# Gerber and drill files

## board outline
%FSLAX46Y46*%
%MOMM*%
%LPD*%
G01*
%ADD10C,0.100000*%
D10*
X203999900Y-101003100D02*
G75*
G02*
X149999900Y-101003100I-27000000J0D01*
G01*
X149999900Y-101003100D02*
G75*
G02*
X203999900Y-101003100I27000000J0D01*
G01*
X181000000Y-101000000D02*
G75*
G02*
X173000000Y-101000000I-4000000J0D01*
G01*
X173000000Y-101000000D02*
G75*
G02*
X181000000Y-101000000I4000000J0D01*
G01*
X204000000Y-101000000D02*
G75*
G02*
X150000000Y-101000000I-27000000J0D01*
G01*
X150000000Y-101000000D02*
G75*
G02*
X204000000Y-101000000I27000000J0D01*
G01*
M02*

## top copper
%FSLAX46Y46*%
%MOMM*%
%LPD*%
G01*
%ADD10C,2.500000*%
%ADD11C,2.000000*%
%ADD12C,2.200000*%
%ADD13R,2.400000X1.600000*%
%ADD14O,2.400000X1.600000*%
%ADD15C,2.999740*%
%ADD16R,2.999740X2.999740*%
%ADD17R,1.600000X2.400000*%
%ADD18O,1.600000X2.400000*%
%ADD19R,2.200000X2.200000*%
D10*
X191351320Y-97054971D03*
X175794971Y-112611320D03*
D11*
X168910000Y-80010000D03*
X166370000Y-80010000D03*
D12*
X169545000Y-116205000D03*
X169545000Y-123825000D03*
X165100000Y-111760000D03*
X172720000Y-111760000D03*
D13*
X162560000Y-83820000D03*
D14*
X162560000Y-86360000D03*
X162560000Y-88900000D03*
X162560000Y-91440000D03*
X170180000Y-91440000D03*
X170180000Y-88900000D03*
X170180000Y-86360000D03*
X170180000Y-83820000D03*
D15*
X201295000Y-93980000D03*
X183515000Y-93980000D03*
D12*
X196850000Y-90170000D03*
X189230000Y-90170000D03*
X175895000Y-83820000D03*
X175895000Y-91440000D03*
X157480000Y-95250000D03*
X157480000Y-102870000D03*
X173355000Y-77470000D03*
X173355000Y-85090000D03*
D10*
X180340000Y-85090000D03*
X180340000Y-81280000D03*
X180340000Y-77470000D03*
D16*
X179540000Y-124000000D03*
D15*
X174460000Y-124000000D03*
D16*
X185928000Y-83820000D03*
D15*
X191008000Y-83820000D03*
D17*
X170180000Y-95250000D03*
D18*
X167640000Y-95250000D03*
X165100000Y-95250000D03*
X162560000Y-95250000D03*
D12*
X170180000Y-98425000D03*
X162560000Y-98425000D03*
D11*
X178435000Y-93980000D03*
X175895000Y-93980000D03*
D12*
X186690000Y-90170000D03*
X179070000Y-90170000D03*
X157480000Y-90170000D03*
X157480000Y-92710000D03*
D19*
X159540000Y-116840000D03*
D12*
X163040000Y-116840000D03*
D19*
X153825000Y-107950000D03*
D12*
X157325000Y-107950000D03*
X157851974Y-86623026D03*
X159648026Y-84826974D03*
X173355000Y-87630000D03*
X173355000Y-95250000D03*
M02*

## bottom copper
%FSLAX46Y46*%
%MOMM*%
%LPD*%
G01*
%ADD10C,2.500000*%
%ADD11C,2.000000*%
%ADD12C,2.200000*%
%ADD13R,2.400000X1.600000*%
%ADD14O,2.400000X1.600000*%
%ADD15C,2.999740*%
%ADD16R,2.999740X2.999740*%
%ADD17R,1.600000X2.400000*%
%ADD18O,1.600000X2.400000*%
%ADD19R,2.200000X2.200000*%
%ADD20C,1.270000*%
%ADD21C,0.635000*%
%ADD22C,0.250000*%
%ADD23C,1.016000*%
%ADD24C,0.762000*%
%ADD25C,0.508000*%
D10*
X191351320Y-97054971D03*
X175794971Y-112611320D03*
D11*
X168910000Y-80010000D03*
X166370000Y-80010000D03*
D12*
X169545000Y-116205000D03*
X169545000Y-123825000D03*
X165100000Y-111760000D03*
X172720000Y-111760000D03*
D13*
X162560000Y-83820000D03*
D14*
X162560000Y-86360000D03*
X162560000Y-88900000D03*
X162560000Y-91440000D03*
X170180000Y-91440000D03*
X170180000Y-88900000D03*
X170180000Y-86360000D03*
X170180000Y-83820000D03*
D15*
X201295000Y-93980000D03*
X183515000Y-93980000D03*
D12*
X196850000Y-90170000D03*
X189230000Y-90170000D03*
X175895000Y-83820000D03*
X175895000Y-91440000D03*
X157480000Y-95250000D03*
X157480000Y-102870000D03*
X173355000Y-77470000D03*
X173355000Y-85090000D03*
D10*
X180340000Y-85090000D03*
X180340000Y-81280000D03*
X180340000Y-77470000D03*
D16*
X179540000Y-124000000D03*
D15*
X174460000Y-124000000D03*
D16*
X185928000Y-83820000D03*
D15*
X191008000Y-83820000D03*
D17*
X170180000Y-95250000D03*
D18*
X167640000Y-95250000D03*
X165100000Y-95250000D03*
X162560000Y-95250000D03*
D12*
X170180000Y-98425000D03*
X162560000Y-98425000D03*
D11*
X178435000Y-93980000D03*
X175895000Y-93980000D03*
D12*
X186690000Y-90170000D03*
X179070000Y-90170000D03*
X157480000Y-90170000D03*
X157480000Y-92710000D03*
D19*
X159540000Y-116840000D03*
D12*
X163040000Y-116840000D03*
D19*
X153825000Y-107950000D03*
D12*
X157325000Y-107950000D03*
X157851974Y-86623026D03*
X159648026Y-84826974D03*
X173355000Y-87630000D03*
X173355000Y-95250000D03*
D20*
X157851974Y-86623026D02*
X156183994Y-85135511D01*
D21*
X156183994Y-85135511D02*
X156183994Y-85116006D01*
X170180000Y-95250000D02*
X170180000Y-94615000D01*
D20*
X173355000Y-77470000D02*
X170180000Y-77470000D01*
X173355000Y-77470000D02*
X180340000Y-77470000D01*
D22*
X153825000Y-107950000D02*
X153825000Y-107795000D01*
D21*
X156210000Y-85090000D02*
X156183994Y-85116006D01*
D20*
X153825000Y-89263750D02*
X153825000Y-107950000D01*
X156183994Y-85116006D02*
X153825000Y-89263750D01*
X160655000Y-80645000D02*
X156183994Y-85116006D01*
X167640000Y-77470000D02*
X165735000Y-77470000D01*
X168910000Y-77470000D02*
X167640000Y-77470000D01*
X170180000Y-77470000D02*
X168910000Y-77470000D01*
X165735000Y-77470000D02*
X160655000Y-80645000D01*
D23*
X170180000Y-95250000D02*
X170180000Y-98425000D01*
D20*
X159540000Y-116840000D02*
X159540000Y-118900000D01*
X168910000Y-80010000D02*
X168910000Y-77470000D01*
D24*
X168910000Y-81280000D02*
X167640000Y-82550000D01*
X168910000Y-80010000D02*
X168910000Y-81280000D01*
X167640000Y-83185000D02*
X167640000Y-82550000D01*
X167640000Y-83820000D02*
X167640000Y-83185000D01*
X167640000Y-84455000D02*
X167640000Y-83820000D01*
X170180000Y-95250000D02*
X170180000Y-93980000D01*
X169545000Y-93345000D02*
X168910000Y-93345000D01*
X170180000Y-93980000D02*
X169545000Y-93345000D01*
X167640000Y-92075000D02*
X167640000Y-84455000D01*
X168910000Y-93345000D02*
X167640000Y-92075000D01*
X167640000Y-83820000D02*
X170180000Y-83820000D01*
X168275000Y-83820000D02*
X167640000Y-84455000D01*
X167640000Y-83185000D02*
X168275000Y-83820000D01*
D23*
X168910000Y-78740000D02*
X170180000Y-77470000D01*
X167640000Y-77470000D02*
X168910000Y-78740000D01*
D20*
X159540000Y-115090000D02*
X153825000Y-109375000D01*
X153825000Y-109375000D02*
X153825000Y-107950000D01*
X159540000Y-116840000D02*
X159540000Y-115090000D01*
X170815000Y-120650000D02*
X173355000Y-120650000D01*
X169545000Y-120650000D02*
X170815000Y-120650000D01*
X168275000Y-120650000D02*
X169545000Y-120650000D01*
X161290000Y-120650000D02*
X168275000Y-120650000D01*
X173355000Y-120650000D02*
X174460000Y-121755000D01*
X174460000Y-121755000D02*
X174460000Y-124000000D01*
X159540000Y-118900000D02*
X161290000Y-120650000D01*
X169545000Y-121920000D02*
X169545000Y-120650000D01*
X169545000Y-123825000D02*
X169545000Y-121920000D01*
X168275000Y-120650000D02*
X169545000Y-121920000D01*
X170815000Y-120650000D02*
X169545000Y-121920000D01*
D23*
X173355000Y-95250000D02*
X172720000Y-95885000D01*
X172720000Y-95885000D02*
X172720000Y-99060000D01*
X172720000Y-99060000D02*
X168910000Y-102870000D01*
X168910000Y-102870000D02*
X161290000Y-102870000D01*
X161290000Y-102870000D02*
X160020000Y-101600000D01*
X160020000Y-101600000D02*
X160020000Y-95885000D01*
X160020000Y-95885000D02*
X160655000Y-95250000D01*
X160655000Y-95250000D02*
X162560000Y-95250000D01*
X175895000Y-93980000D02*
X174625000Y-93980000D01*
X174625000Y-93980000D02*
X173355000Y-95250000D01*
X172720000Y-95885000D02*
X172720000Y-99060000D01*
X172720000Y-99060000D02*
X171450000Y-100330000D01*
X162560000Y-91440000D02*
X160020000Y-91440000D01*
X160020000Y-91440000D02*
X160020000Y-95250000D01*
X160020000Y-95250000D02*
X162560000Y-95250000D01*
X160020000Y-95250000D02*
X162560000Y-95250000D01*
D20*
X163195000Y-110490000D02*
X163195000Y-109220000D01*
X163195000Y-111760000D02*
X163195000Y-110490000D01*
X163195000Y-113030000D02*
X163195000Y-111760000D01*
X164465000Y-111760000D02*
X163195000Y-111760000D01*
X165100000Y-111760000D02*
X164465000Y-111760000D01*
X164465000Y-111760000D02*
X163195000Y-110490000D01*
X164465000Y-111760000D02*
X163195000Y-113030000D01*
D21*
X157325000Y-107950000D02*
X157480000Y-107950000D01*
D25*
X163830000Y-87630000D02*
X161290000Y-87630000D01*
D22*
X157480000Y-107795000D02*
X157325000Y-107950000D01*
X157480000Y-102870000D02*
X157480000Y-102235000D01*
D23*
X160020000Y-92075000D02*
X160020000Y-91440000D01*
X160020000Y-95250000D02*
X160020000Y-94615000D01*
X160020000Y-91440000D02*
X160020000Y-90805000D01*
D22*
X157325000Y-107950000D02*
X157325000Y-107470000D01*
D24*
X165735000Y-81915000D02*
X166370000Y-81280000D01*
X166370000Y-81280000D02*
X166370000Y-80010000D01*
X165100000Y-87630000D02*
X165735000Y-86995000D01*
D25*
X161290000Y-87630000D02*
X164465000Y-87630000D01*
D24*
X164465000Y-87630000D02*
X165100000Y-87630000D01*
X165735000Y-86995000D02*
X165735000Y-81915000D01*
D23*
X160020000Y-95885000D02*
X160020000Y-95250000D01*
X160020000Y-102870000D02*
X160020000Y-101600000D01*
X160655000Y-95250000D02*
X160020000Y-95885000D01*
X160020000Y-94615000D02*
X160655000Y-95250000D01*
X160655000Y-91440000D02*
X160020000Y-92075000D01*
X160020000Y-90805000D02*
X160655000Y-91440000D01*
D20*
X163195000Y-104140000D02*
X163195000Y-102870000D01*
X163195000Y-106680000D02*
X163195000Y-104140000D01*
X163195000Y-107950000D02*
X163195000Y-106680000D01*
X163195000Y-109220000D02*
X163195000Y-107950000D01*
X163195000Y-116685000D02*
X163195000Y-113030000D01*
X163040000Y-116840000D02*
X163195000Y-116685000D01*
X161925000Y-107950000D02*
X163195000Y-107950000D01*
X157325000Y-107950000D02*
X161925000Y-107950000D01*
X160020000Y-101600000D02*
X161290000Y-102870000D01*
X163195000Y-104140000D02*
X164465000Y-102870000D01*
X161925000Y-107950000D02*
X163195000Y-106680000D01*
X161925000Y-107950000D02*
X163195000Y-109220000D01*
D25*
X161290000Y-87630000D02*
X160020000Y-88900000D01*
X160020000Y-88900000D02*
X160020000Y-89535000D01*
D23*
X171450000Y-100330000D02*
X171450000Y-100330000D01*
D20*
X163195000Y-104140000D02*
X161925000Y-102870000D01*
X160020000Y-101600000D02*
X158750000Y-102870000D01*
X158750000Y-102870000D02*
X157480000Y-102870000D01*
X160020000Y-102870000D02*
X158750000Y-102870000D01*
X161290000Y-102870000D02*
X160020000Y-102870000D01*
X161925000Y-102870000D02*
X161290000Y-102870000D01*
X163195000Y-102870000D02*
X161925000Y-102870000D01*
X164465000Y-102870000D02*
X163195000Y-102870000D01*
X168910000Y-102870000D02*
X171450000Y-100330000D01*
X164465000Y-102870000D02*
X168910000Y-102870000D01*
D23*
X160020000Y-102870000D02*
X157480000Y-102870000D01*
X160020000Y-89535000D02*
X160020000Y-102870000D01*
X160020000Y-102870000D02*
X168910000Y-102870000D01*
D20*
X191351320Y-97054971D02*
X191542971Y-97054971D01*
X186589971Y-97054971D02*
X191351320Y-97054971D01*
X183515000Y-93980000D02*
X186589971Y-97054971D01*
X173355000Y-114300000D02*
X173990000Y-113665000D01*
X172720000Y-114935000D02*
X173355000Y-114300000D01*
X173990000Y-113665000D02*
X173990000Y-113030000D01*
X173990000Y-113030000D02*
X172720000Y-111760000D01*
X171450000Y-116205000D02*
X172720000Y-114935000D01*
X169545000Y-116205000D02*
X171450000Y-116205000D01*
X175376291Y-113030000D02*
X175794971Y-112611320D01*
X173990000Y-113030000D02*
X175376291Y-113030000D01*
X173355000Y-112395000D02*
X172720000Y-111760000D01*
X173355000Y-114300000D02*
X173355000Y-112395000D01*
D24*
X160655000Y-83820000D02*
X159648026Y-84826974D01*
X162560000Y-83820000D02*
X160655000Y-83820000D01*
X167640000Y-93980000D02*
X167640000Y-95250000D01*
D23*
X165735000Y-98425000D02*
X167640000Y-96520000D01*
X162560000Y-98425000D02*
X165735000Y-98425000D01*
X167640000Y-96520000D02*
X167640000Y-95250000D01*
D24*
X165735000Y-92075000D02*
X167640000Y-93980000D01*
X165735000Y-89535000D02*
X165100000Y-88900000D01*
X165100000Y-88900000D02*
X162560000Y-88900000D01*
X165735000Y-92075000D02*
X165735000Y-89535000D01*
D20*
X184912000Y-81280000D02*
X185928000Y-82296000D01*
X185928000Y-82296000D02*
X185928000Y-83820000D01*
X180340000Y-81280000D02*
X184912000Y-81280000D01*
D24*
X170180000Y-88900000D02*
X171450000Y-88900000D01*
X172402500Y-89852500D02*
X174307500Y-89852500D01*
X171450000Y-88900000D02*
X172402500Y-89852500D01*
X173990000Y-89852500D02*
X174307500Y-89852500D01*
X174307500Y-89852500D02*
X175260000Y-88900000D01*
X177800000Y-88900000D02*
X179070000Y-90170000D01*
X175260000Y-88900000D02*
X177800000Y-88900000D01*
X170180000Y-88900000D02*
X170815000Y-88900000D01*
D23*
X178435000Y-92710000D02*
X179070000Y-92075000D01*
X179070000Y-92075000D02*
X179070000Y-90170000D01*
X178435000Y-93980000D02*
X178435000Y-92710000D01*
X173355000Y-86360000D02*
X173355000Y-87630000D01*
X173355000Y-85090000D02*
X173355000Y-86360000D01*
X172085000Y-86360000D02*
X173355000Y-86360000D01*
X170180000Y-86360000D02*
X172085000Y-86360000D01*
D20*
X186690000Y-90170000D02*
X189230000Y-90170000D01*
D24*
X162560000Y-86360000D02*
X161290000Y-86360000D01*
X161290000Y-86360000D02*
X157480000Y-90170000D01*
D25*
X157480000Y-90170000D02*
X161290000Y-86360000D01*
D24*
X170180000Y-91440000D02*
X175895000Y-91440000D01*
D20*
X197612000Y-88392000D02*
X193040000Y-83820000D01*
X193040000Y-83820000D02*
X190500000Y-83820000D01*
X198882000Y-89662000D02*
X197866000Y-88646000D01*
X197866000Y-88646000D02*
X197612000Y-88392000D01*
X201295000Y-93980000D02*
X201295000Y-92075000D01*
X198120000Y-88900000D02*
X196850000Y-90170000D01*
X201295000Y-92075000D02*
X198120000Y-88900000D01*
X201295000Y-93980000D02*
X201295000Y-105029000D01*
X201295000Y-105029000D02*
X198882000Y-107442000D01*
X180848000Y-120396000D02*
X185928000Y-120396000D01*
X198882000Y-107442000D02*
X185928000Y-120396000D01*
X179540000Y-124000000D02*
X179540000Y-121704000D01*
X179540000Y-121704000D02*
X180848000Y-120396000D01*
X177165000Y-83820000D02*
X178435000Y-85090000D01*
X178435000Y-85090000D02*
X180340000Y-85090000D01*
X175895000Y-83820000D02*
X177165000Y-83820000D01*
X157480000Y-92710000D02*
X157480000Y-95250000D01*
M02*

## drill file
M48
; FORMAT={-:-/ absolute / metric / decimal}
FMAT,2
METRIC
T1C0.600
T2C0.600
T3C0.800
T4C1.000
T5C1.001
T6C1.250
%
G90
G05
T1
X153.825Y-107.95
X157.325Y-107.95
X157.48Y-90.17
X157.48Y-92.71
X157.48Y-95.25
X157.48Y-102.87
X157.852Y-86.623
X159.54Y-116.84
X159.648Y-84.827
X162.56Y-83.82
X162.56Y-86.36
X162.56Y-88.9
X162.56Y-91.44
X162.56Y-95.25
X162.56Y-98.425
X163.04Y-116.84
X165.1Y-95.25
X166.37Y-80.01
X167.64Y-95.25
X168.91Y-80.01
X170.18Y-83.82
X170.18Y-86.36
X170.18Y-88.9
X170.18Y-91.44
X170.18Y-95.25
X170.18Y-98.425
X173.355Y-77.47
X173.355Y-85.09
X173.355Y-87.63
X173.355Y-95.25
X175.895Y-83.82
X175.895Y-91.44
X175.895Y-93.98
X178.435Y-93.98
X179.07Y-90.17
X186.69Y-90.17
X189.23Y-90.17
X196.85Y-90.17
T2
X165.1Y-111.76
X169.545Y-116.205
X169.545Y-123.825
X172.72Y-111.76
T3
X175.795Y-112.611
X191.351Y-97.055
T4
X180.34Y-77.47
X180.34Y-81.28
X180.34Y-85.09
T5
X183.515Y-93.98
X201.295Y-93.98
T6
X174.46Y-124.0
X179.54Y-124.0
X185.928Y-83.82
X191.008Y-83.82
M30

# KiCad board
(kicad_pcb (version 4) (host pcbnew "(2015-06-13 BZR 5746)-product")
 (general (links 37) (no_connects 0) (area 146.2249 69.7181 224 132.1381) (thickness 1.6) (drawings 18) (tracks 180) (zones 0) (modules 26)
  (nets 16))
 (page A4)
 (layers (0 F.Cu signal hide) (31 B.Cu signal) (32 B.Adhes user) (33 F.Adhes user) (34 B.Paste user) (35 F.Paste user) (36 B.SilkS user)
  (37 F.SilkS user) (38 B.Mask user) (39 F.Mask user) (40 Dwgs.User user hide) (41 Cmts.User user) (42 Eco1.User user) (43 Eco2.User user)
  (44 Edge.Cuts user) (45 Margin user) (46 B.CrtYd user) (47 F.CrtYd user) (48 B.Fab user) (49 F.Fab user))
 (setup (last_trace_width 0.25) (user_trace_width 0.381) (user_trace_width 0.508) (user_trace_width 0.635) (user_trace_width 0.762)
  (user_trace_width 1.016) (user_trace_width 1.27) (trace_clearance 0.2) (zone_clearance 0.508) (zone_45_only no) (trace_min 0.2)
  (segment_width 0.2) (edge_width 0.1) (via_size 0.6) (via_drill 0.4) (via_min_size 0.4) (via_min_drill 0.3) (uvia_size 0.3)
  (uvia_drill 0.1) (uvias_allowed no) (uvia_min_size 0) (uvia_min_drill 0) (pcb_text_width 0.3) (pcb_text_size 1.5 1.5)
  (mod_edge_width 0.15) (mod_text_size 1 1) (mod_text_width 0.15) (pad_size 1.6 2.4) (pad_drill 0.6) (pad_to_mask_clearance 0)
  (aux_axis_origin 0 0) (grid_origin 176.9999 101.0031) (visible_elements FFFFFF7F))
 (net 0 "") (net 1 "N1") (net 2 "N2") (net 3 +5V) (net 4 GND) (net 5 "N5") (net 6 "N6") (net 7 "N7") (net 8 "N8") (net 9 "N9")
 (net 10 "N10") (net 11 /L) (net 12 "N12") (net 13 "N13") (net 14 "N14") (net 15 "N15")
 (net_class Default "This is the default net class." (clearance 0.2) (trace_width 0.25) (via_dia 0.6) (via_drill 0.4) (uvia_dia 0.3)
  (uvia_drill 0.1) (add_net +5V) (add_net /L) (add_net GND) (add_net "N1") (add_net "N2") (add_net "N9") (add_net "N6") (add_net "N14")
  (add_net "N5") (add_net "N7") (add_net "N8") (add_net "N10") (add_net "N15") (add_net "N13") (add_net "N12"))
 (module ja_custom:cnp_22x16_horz (layer F.Cu) (at 189.23 110.49 225)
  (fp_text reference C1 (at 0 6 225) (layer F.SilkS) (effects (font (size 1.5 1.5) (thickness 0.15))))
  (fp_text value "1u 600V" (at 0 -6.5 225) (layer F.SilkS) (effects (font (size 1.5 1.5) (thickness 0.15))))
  (pad 1 thru_hole circle (at -11 8 225) (size 2.5 2.5) (drill 0.8) (layers *.Cu *.Mask F.SilkS) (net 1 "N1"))
  (pad 2 thru_hole circle (at 11 8 225) (size 2.5 2.5) (drill 0.8) (layers *.Cu *.Mask F.SilkS) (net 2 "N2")))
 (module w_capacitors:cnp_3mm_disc (layer F.Cu) (at 167.64 80.01 180)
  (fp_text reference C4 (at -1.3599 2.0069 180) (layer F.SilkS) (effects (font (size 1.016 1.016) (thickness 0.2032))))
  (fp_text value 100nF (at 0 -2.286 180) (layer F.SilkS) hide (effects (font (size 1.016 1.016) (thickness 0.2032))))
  (pad 1 thru_hole circle (at -1.27 0 180) (size 2 2) (drill 0.6) (layers *.Cu *.Mask F.SilkS) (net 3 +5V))
  (pad 2 thru_hole circle (at 1.27 0 180) (size 2 2) (drill 0.6) (layers *.Cu *.Mask F.SilkS) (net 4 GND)))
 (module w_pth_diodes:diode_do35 (layer F.Cu) (at 169.545 120.015 270)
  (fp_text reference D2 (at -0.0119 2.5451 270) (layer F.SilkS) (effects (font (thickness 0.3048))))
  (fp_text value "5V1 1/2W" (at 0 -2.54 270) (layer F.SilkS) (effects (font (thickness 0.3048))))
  (pad 1 thru_hole circle (at -3.81 0 270) (size 2.2 2.2) (drill 0.6001) (layers *.Cu *.Mask F.SilkS) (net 2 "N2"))
  (pad 2 thru_hole circle (at 3.81 0 270) (size 2.2 2.2) (drill 0.6001) (layers *.Cu *.Mask F.SilkS) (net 3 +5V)))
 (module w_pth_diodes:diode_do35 (layer F.Cu) (at 168.91 111.76)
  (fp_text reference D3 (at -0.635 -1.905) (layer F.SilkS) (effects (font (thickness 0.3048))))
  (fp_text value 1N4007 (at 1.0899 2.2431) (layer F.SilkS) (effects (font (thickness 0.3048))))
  (pad 1 thru_hole circle (at -3.81 0) (size 2.2 2.2) (drill 0.6001) (layers *.Cu *.Mask F.SilkS) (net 4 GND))
  (pad 2 thru_hole circle (at 3.81 0) (size 2.2 2.2) (drill 0.6001) (layers *.Cu *.Mask F.SilkS) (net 2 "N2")))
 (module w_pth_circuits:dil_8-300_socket (layer F.Cu) (at 166.37 87.63 270)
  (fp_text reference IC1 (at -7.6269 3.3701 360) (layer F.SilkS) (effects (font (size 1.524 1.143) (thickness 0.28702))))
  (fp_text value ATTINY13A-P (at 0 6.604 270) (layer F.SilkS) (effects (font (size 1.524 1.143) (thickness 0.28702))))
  (pad 1 thru_hole rect (at -3.81 3.81 270) (size 1.6 2.4) (drill 0.6) (layers *.Cu *.Mask F.SilkS) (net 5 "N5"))
  (pad 2 thru_hole oval (at -1.27 3.81 270) (size 1.6 2.4) (drill 0.6) (layers *.Cu *.Mask F.SilkS) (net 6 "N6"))
  (pad 3 thru_hole oval (at 1.27 3.81 270) (size 1.6 2.4) (drill 0.6) (layers *.Cu *.Mask F.SilkS) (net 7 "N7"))
  (pad 4 thru_hole oval (at 3.81 3.81 270) (size 1.6 2.4) (drill 0.6) (layers *.Cu *.Mask F.SilkS) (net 4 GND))
  (pad 5 thru_hole oval (at 3.81 -3.81 270) (size 1.6 2.4) (drill 0.6) (layers *.Cu *.Mask F.SilkS) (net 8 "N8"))
  (pad 6 thru_hole oval (at 1.27 -3.81 270) (size 1.6 2.4) (drill 0.6) (layers *.Cu *.Mask F.SilkS) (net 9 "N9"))
  (pad 7 thru_hole oval (at -1.27 -3.81 270) (size 1.6 2.4) (drill 0.6) (layers *.Cu *.Mask F.SilkS) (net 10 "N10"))
  (pad 8 thru_hole oval (at -3.81 -3.81 270) (size 1.6 2.4) (drill 0.6) (layers *.Cu *.Mask F.SilkS) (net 3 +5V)))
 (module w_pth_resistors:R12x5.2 (layer F.Cu) (at 192.405 93.98 180) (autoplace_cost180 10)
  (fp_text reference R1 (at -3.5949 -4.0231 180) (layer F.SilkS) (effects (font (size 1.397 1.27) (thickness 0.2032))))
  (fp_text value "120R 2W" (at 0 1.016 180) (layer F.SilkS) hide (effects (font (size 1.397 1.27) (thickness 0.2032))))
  (pad 1 thru_hole circle (at -8.89 0 180) (size 2.99974 2.99974) (drill 1.00076) (layers *.Cu *.Mask F.SilkS) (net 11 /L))
  (pad 2 thru_hole circle (at 8.89 0 180) (size 2.99974 2.99974) (drill 1.00076) (layers *.Cu *.Mask F.SilkS) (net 1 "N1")))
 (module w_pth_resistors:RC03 (layer F.Cu) (at 193.04 90.17 180) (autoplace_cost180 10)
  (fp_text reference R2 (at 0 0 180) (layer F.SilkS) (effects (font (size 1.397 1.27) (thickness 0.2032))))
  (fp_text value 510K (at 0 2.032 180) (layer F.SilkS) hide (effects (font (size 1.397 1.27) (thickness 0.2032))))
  (pad 1 thru_hole circle (at -3.81 0 180) (size 2.2 2.2) (drill 0.6) (layers *.Cu *.Mask F.SilkS) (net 11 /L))
  (pad 2 thru_hole circle (at 3.81 0 180) (size 2.2 2.2) (drill 0.6) (layers *.Cu *.Mask F.SilkS) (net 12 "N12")))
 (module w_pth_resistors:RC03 (layer F.Cu) (at 175.895 87.63 270) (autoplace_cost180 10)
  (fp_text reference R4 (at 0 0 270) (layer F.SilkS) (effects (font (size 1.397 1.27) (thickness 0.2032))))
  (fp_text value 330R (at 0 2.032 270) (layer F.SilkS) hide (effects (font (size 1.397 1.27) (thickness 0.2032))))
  (pad 1 thru_hole circle (at -3.81 0 270) (size 2.2 2.2) (drill 0.6) (layers *.Cu *.Mask F.SilkS) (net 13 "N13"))
  (pad 2 thru_hole circle (at 3.81 0 270) (size 2.2 2.2) (drill 0.6) (layers *.Cu *.Mask F.SilkS) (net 8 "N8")))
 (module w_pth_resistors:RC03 (layer F.Cu) (at 157.48 99.06 270) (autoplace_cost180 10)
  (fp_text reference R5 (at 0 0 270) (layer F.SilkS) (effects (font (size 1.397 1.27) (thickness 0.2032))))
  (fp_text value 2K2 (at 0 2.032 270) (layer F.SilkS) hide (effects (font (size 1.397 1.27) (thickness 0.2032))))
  (pad 1 thru_hole circle (at -3.81 0 270) (size 2.2 2.2) (drill 0.6) (layers *.Cu *.Mask F.SilkS) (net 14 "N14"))
  (pad 2 thru_hole circle (at 3.81 0 270) (size 2.2 2.2) (drill 0.6) (layers *.Cu *.Mask F.SilkS) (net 4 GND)))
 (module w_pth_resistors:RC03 (layer F.Cu) (at 173.355 81.28 270) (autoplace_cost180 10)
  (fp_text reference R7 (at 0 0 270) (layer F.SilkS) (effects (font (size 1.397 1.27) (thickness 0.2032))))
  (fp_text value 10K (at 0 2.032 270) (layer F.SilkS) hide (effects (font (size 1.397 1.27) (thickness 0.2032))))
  (pad 1 thru_hole circle (at -3.81 0 270) (size 2.2 2.2) (drill 0.6) (layers *.Cu *.Mask F.SilkS) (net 3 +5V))
  (pad 2 thru_hole circle (at 3.81 0 270) (size 2.2 2.2) (drill 0.6) (layers *.Cu *.Mask F.SilkS) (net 10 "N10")))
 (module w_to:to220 (layer F.Cu) (at 180.34 81.28 270)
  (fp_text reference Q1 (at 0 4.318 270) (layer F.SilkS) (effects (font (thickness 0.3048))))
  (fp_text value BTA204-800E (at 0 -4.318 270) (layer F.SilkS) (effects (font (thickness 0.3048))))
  (pad 1 thru_hole circle (at 3.81 0 270) (size 2.5 2.5) (drill 1) (layers *.Cu *.Mask F.SilkS) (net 13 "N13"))
  (pad 2 thru_hole circle (at 0 0 270) (size 2.5 2.5) (drill 1) (layers *.Cu *.Mask F.SilkS) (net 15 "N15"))
  (pad 3 thru_hole circle (at -3.81 0 270) (size 2.5 2.5) (drill 1) (layers *.Cu *.Mask F.SilkS) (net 3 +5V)))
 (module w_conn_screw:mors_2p (layer F.Cu) (at 177 124 180)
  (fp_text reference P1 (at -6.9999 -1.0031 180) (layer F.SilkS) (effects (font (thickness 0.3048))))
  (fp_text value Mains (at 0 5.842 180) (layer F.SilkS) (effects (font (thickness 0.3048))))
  (pad 1 thru_hole rect (at -2.54 0 180) (size 2.99974 2.99974) (drill 1.24968) (layers *.Cu *.Mask F.SilkS) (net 11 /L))
  (pad 2 thru_hole circle (at 2.54 0 180) (size 2.99974 2.99974) (drill 1.24968) (layers *.Cu *.Mask F.SilkS) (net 3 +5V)))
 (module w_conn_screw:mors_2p (layer F.Cu) (at 188.468 83.82)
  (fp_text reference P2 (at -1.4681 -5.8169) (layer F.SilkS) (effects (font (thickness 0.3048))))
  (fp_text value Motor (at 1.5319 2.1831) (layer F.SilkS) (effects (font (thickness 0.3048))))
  (pad 1 thru_hole rect (at -2.54 0) (size 2.99974 2.99974) (drill 1.24968) (layers *.Cu *.Mask F.SilkS) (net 15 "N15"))
  (pad 2 thru_hole circle (at 2.54 0) (size 2.99974 2.99974) (drill 1.24968) (layers *.Cu *.Mask F.SilkS) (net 11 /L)))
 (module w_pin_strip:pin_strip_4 (layer F.Cu) (at 166.37 95.25 180)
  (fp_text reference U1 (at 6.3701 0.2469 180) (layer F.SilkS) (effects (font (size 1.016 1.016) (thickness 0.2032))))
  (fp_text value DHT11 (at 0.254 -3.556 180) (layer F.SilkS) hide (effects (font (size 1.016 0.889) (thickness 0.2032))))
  (pad 1 thru_hole rect (at -3.81 0 180) (size 1.6 2.4) (drill 0.6) (layers *.Cu *.Mask F.SilkS) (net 3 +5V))
  (pad 2 thru_hole oval (at -1.27 0 180) (size 1.6 2.4) (drill 0.6) (layers *.Cu *.Mask F.SilkS) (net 7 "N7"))
  (pad 3 thru_hole oval (at 1.27 0 180) (size 1.6 2.4) (drill 0.6) (layers *.Cu *.Mask F.SilkS))
  (pad 4 thru_hole oval (at 3.81 0 180) (size 1.6 2.4) (drill 0.6) (layers *.Cu *.Mask F.SilkS) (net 4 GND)))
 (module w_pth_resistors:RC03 (layer F.Cu) (at 166.37 98.425 180) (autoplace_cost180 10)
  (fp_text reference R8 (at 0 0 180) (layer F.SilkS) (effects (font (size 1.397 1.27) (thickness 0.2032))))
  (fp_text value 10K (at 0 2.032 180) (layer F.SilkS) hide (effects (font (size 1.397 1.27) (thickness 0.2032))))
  (pad 1 thru_hole circle (at -3.81 0 180) (size 2.2 2.2) (drill 0.6) (layers *.Cu *.Mask F.SilkS) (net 3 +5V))
  (pad 2 thru_hole circle (at 3.81 0 180) (size 2.2 2.2) (drill 0.6) (layers *.Cu *.Mask F.SilkS) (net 7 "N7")))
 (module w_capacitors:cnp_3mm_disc (layer F.Cu) (at 177.165 93.98 180)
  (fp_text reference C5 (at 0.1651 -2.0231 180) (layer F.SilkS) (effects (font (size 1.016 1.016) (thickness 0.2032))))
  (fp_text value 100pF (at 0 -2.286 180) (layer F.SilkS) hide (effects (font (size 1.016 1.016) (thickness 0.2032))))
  (pad 1 thru_hole circle (at -1.27 0 180) (size 2 2) (drill 0.6) (layers *.Cu *.Mask F.SilkS) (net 9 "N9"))
  (pad 2 thru_hole circle (at 1.27 0 180) (size 2 2) (drill 0.6) (layers *.Cu *.Mask F.SilkS) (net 4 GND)))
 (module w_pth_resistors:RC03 (layer F.Cu) (at 182.88 90.17 180) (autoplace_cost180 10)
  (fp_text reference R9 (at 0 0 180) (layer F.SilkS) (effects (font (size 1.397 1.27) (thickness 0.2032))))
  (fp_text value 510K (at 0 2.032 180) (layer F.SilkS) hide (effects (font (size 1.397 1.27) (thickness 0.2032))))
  (pad 1 thru_hole circle (at -3.81 0 180) (size 2.2 2.2) (drill 0.6) (layers *.Cu *.Mask F.SilkS) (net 12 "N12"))
  (pad 2 thru_hole circle (at 3.81 0 180) (size 2.2 2.2) (drill 0.6) (layers *.Cu *.Mask F.SilkS) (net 9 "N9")))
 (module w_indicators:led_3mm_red (layer F.Cu) (at 157.48 91.44)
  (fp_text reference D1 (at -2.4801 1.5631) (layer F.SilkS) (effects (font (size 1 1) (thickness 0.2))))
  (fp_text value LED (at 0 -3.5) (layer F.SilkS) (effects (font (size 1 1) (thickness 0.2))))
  (pad 1 thru_hole circle (at 0 -1.27) (size 2.2 2.2) (drill 0.6) (layers *.Cu *.Mask F.SilkS) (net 6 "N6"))
  (pad 2 thru_hole circle (at 0 1.27) (size 2.2 2.2) (drill 0.6) (layers *.Cu *.Mask F.SilkS) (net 14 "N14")))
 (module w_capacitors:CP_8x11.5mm (layer F.Cu) (at 161.29 116.84 270)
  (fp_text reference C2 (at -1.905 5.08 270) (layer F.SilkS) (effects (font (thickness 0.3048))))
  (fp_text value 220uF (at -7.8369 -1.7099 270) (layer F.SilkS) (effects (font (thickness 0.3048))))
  (pad 1 thru_hole rect (at 0 1.75 270) (size 2.2 2.2) (drill 0.6) (layers *.Cu *.Mask F.SilkS) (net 3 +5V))
  (pad 2 thru_hole circle (at 0 -1.75 270) (size 2.2 2.2) (drill 0.6) (layers *.Cu *.Mask F.SilkS) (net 4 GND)))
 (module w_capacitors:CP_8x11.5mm (layer F.Cu) (at 155.575 107.95 270)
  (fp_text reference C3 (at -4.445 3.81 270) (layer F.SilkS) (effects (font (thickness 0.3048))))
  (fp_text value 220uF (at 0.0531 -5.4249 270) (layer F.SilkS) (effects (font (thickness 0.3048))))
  (pad 1 thru_hole rect (at 0 1.75 270) (size 2.2 2.2) (drill 0.6) (layers *.Cu *.Mask F.SilkS) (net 3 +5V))
  (pad 2 thru_hole circle (at 0 -1.75 270) (size 2.2 2.2) (drill 0.6) (layers *.Cu *.Mask F.SilkS) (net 4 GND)))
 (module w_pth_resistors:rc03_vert (layer F.Cu) (at 158.75 85.725 45)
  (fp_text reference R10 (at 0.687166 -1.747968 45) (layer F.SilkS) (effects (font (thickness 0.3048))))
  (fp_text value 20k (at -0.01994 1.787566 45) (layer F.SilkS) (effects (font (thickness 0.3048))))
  (pad 1 thru_hole circle (at -1.270001 0 45) (size 2.2 2.2) (drill 0.6) (layers *.Cu *.Mask F.SilkS) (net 3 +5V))
  (pad 2 thru_hole circle (at 1.27 0 45) (size 2.2 2.2) (drill 0.6) (layers *.Cu *.Mask F.SilkS) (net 5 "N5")))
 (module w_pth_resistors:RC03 (layer F.Cu) (at 173.355 91.44 270) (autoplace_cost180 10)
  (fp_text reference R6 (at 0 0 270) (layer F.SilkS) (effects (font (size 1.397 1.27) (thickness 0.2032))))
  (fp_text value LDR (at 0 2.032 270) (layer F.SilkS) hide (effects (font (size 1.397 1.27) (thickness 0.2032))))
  (pad 1 thru_hole circle (at -3.81 0 270) (size 2.2 2.2) (drill 0.6) (layers *.Cu *.Mask F.SilkS) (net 10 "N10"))
  (pad 2 thru_hole circle (at 3.81 0 270) (size 2.2 2.2) (drill 0.6) (layers *.Cu *.Mask F.SilkS) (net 4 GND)))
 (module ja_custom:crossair (layer F.Cu) (at 202.9999 75.0031)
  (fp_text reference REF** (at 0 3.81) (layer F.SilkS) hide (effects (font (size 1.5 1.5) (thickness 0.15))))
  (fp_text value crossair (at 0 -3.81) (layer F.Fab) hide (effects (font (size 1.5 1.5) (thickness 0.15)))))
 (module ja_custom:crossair (layer F.Cu) (at 150.9999 75.0031)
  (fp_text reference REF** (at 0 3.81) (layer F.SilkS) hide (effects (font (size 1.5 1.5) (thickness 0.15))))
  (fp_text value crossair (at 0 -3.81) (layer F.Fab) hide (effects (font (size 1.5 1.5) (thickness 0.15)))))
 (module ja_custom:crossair (layer F.Cu) (at 150.9999 127.0031)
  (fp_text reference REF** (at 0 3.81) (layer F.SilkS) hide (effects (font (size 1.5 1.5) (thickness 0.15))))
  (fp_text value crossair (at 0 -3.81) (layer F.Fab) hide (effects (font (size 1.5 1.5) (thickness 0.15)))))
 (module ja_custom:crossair (layer F.Cu) (at 202.9999 127.0031)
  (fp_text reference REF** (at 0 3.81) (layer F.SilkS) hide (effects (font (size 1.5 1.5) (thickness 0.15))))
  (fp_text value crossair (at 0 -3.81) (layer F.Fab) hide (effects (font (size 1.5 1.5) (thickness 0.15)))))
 (gr_circle (center 176.9999 101.0031) (end 203.9999 101.0031) (layer Edge.Cuts) (width 0.1))
 (gr_circle (center 177 101) (end 181 101) (layer Edge.Cuts) (width 0.1))
 (gr_circle (center 177 101) (end 204 101) (layer Edge.Cuts) (width 0.1))
 (segment (start 157.851974 86.623026) (end 156.183994 85.135511) (width 1.27) (layer B.Cu) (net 3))
 (segment (start 156.183994 85.135511) (end 156.183994 85.116006) (width 0.635) (layer B.Cu) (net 3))
 (segment (start 170.18 95.25) (end 170.18 94.615) (width 0.635) (layer B.Cu) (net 3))
 (segment (start 173.355 77.47) (end 170.18 77.47) (width 1.27) (layer B.Cu) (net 3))
 (segment (start 173.355 77.47) (end 180.34 77.47) (width 1.27) (layer B.Cu) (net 3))
 (segment (start 153.825 107.95) (end 153.825 107.795) (width 0.25) (layer B.Cu) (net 3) (status 30))
 (segment (start 156.21 85.09) (end 156.183994 85.116006) (width 0.635) (layer B.Cu) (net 3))
 (segment (start 153.825 89.26375) (end 153.825 107.95) (width 1.27) (layer B.Cu) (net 3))
 (segment (start 156.183994 85.116006) (end 153.825 89.26375) (width 1.27) (layer B.Cu) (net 3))
 (segment (start 160.655 80.645) (end 156.183994 85.116006) (width 1.27) (layer B.Cu) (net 3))
 (segment (start 167.64 77.47) (end 165.735 77.47) (width 1.27) (layer B.Cu) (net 3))
 (segment (start 168.91 77.47) (end 167.64 77.47) (width 1.27) (layer B.Cu) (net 3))
 (segment (start 170.18 77.47) (end 168.91 77.47) (width 1.27) (layer B.Cu) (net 3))
 (segment (start 165.735 77.47) (end 160.655 80.645) (width 1.27) (layer B.Cu) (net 3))
 (segment (start 170.18 95.25) (end 170.18 98.425) (width 1.016) (layer B.Cu) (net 3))
 (segment (start 159.54 116.84) (end 159.54 118.9) (width 1.27) (layer B.Cu) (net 3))
 (segment (start 168.91 80.01) (end 168.91 77.47) (width 1.27) (layer B.Cu) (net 3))
 (segment (start 168.91 81.28) (end 167.64 82.55) (width 0.762) (layer B.Cu) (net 3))
 (segment (start 168.91 80.01) (end 168.91 81.28) (width 0.762) (layer B.Cu) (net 3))
 (segment (start 167.64 83.185) (end 167.64 82.55) (width 0.762) (layer B.Cu) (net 3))
 (segment (start 167.64 83.82) (end 167.64 83.185) (width 0.762) (layer B.Cu) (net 3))
 (segment (start 167.64 84.455) (end 167.64 83.82) (width 0.762) (layer B.Cu) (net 3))
 (segment (start 170.18 95.25) (end 170.18 93.98) (width 0.762) (layer B.Cu) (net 3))
 (segment (start 169.545 93.345) (end 168.91 93.345) (width 0.762) (layer B.Cu) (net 3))
 (segment (start 170.18 93.98) (end 169.545 93.345) (width 0.762) (layer B.Cu) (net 3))
 (segment (start 167.64 92.075) (end 167.64 84.455) (width 0.762) (layer B.Cu) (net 3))
 (segment (start 168.91 93.345) (end 167.64 92.075) (width 0.762) (layer B.Cu) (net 3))
 (segment (start 167.64 83.82) (end 170.18 83.82) (width 0.762) (layer B.Cu) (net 3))
 (segment (start 168.275 83.82) (end 167.64 84.455) (width 0.762) (layer B.Cu) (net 3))
 (segment (start 167.64 83.185) (end 168.275 83.82) (width 0.762) (layer B.Cu) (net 3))
 (segment (start 168.91 78.74) (end 170.18 77.47) (width 1.016) (layer B.Cu) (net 3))
 (segment (start 167.64 77.47) (end 168.91 78.74) (width 1.016) (layer B.Cu) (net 3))
 (segment (start 159.54 115.09) (end 153.825 109.375) (width 1.27) (layer B.Cu) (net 3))
 (segment (start 153.825 109.375) (end 153.825 107.95) (width 1.27) (layer B.Cu) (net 3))
 (segment (start 159.54 116.84) (end 159.54 115.09) (width 1.27) (layer B.Cu) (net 3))
 (segment (start 170.815 120.65) (end 173.355 120.65) (width 1.27) (layer B.Cu) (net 3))
 (segment (start 169.545 120.65) (end 170.815 120.65) (width 1.27) (layer B.Cu) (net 3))
 (segment (start 168.275 120.65) (end 169.545 120.65) (width 1.27) (layer B.Cu) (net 3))
 (segment (start 161.29 120.65) (end 168.275 120.65) (width 1.27) (layer B.Cu) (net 3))
 (segment (start 173.355 120.65) (end 174.46 121.755) (width 1.27) (layer B.Cu) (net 3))
 (segment (start 174.46 121.755) (end 174.46 124) (width 1.27) (layer B.Cu) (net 3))
 (segment (start 159.54 118.9) (end 161.29 120.65) (width 1.27) (layer B.Cu) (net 3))
 (segment (start 169.545 121.92) (end 169.545 120.65) (width 1.27) (layer B.Cu) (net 3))
 (segment (start 169.545 123.825) (end 169.545 121.92) (width 1.27) (layer B.Cu) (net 3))
 (segment (start 168.275 120.65) (end 169.545 121.92) (width 1.27) (layer B.Cu) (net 3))
 (segment (start 170.815 120.65) (end 169.545 121.92) (width 1.27) (layer B.Cu) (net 3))
 (segment (start 173.355 95.25) (end 172.72 95.885) (width 1.016) (layer B.Cu) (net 4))
 (segment (start 172.72 95.885) (end 172.72 99.06) (width 1.016) (layer B.Cu) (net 4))
 (segment (start 172.72 99.06) (end 168.91 102.87) (width 1.016) (layer B.Cu) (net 4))
 (segment (start 168.91 102.87) (end 161.29 102.87) (width 1.016) (layer B.Cu) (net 4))
 (segment (start 161.29 102.87) (end 160.02 101.6) (width 1.016) (layer B.Cu) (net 4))
 (segment (start 160.02 101.6) (end 160.02 95.885) (width 1.016) (layer B.Cu) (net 4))
 (segment (start 160.02 95.885) (end 160.655 95.25) (width 1.016) (layer B.Cu) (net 4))
 (segment (start 160.655 95.25) (end 162.56 95.25) (width 1.016) (layer B.Cu) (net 4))
 (segment (start 175.895 93.98) (end 174.625 93.98) (width 1.016) (layer B.Cu) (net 4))
 (segment (start 174.625 93.98) (end 173.355 95.25) (width 1.016) (layer B.Cu) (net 4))
 (segment (start 172.72 95.885) (end 172.72 99.06) (width 1.016) (layer B.Cu) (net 4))
 (segment (start 172.72 99.06) (end 171.45 100.33) (width 1.016) (layer B.Cu) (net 4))
 (segment (start 162.56 91.44) (end 160.02 91.44) (width 1.016) (layer B.Cu) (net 4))
 (segment (start 160.02 91.44) (end 160.02 95.25) (width 1.016) (layer B.Cu) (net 4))
 (segment (start 160.02 95.25) (end 162.56 95.25) (width 1.016) (layer B.Cu) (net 4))
 (segment (start 160.02 95.25) (end 162.56 95.25) (width 1.016) (layer B.Cu) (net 4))
 (segment (start 163.195 110.49) (end 163.195 109.22) (width 1.27) (layer B.Cu) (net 4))
 (segment (start 163.195 111.76) (end 163.195 110.49) (width 1.27) (layer B.Cu) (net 4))
 (segment (start 163.195 113.03) (end 163.195 111.76) (width 1.27) (layer B.Cu) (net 4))
 (segment (start 164.465 111.76) (end 163.195 111.76) (width 1.27) (layer B.Cu) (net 4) (status 10))
 (segment (start 165.1 111.76) (end 164.465 111.76) (width 1.27) (layer B.Cu) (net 4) (status 10))
 (segment (start 164.465 111.76) (end 163.195 110.49) (width 1.27) (layer B.Cu) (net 4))
 (segment (start 164.465 111.76) (end 163.195 113.03) (width 1.27) (layer B.Cu) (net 4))
 (segment (start 157.325 107.95) (end 157.48 107.95) (width 0.635) (layer B.Cu) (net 4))
 (segment (start 163.83 87.63) (end 161.29 87.63) (width 0.508) (layer B.Cu) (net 4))
 (segment (start 157.48 107.795) (end 157.325 107.95) (width 0.25) (layer B.Cu) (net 4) (status 30))
 (segment (start 157.48 102.87) (end 157.48 102.235) (width 0.25) (layer B.Cu) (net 4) (status 30))
 (segment (start 160.02 92.075) (end 160.02 91.44) (width 1.016) (layer B.Cu) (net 4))
 (segment (start 160.02 95.25) (end 160.02 94.615) (width 1.016) (layer B.Cu) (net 4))
 (segment (start 160.02 91.44) (end 160.02 90.805) (width 1.016) (layer B.Cu) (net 4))
 (segment (start 157.325 107.95) (end 157.325 107.47) (width 0.25) (layer B.Cu) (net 4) (status 30))
 (segment (start 165.735 81.915) (end 166.37 81.28) (width 0.762) (layer B.Cu) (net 4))
 (segment (start 166.37 81.28) (end 166.37 80.01) (width 0.762) (layer B.Cu) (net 4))
 (segment (start 165.1 87.63) (end 165.735 86.995) (width 0.762) (layer B.Cu) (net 4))
 (segment (start 161.29 87.63) (end 164.465 87.63) (width 0.508) (layer B.Cu) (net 4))
 (segment (start 164.465 87.63) (end 165.1 87.63) (width 0.762) (layer B.Cu) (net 4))
 (segment (start 165.735 86.995) (end 165.735 81.915) (width 0.762) (layer B.Cu) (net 4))
 (segment (start 160.02 95.885) (end 160.02 95.25) (width 1.016) (layer B.Cu) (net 4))
 (segment (start 160.02 102.87) (end 160.02 101.6) (width 1.016) (layer B.Cu) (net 4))
 (segment (start 160.655 95.25) (end 160.02 95.885) (width 1.016) (layer B.Cu) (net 4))
 (segment (start 160.02 94.615) (end 160.655 95.25) (width 1.016) (layer B.Cu) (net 4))
 (segment (start 160.655 91.44) (end 160.02 92.075) (width 1.016) (layer B.Cu) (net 4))
 (segment (start 160.02 90.805) (end 160.655 91.44) (width 1.016) (layer B.Cu) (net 4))
 (segment (start 163.195 104.14) (end 163.195 102.87) (width 1.27) (layer B.Cu) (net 4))
 (segment (start 163.195 106.68) (end 163.195 104.14) (width 1.27) (layer B.Cu) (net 4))
 (segment (start 163.195 107.95) (end 163.195 106.68) (width 1.27) (layer B.Cu) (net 4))
 (segment (start 163.195 109.22) (end 163.195 107.95) (width 1.27) (layer B.Cu) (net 4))
 (segment (start 163.195 116.685) (end 163.195 113.03) (width 1.27) (layer B.Cu) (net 4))
 (segment (start 163.04 116.84) (end 163.195 116.685) (width 1.27) (layer B.Cu) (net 4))
 (segment (start 161.925 107.95) (end 163.195 107.95) (width 1.27) (layer B.Cu) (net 4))
 (segment (start 157.325 107.95) (end 161.925 107.95) (width 1.27) (layer B.Cu) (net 4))
 (segment (start 160.02 101.6) (end 161.29 102.87) (width 1.27) (layer B.Cu) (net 4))
 (segment (start 163.195 104.14) (end 164.465 102.87) (width 1.27) (layer B.Cu) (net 4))
 (segment (start 161.925 107.95) (end 163.195 106.68) (width 1.27) (layer B.Cu) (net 4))
 (segment (start 161.925 107.95) (end 163.195 109.22) (width 1.27) (layer B.Cu) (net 4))
 (segment (start 161.29 87.63) (end 160.02 88.9) (width 0.508) (layer B.Cu) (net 4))
 (segment (start 160.02 88.9) (end 160.02 89.535) (width 0.508) (layer B.Cu) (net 4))
 (segment (start 171.45 100.33) (end 171.45 100.33) (width 1.016) (layer B.Cu) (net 4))
 (segment (start 163.195 104.14) (end 161.925 102.87) (width 1.27) (layer B.Cu) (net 4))
 (segment (start 160.02 101.6) (end 158.75 102.87) (width 1.27) (layer B.Cu) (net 4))
 (segment (start 158.75 102.87) (end 157.48 102.87) (width 1.27) (layer B.Cu) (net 4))
 (segment (start 160.02 102.87) (end 158.75 102.87) (width 1.27) (layer B.Cu) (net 4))
 (segment (start 161.29 102.87) (end 160.02 102.87) (width 1.27) (layer B.Cu) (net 4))
 (segment (start 161.925 102.87) (end 161.29 102.87) (width 1.27) (layer B.Cu) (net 4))
 (segment (start 163.195 102.87) (end 161.925 102.87) (width 1.27) (layer B.Cu) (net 4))
 (segment (start 164.465 102.87) (end 163.195 102.87) (width 1.27) (layer B.Cu) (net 4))
 (segment (start 168.91 102.87) (end 171.45 100.33) (width 1.27) (layer B.Cu) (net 4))
 (segment (start 164.465 102.87) (end 168.91 102.87) (width 1.27) (layer B.Cu) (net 4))
 (segment (start 160.02 102.87) (end 157.48 102.87) (width 1.016) (layer B.Cu) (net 4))
 (segment (start 160.02 89.535) (end 160.02 102.87) (width 1.016) (layer B.Cu) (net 4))
 (segment (start 160.02 102.87) (end 168.91 102.87) (width 1.016) (layer B.Cu) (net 4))
 (segment (start 191.35132 97.054971) (end 191.542971 97.054971) (width 1.27) (layer B.Cu) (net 1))
 (segment (start 186.589971 97.054971) (end 191.35132 97.054971) (width 1.27) (layer B.Cu) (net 1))
 (segment (start 183.515 93.98) (end 186.589971 97.054971) (width 1.27) (layer B.Cu) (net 1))
 (segment (start 173.355 114.3) (end 173.99 113.665) (width 1.27) (layer B.Cu) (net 2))
 (segment (start 172.72 114.935) (end 173.355 114.3) (width 1.27) (layer B.Cu) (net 2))
 (segment (start 173.99 113.665) (end 173.99 113.03) (width 1.27) (layer B.Cu) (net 2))
 (segment (start 173.99 113.03) (end 172.72 111.76) (width 1.27) (layer B.Cu) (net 2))
 (segment (start 171.45 116.205) (end 172.72 114.935) (width 1.27) (layer B.Cu) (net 2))
 (segment (start 169.545 116.205) (end 171.45 116.205) (width 1.27) (layer B.Cu) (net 2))
 (segment (start 175.376291 113.03) (end 175.794971 112.61132) (width 1.27) (layer B.Cu) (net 2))
 (segment (start 173.99 113.03) (end 175.376291 113.03) (width 1.27) (layer B.Cu) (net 2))
 (segment (start 173.355 112.395) (end 172.72 111.76) (width 1.27) (layer B.Cu) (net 2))
 (segment (start 173.355 114.3) (end 173.355 112.395) (width 1.27) (layer B.Cu) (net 2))
 (segment (start 160.655 83.82) (end 159.648026 84.826974) (width 0.762) (layer B.Cu) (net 5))
 (segment (start 162.56 83.82) (end 160.655 83.82) (width 0.762) (layer B.Cu) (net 5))
 (segment (start 167.64 93.98) (end 167.64 95.25) (width 0.762) (layer B.Cu) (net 7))
 (segment (start 165.735 98.425) (end 167.64 96.52) (width 1.016) (layer B.Cu) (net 7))
 (segment (start 162.56 98.425) (end 165.735 98.425) (width 1.016) (layer B.Cu) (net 7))
 (segment (start 167.64 96.52) (end 167.64 95.25) (width 1.016) (layer B.Cu) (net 7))
 (segment (start 165.735 92.075) (end 167.64 93.98) (width 0.762) (layer B.Cu) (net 7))
 (segment (start 165.735 89.535) (end 165.1 88.9) (width 0.762) (layer B.Cu) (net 7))
 (segment (start 165.1 88.9) (end 162.56 88.9) (width 0.762) (layer B.Cu) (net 7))
 (segment (start 165.735 92.075) (end 165.735 89.535) (width 0.762) (layer B.Cu) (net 7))
 (segment (start 184.912 81.28) (end 185.928 82.296) (width 1.27) (layer B.Cu) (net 15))
 (segment (start 185.928 82.296) (end 185.928 83.82) (width 1.27) (layer B.Cu) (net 15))
 (segment (start 180.34 81.28) (end 184.912 81.28) (width 1.27) (layer B.Cu) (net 15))
 (segment (start 170.18 88.9) (end 171.45 88.9) (width 0.762) (layer B.Cu) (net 9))
 (segment (start 172.4025 89.8525) (end 174.3075 89.8525) (width 0.762) (layer B.Cu) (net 9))
 (segment (start 171.45 88.9) (end 172.4025 89.8525) (width 0.762) (layer B.Cu) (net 9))
 (segment (start 173.99 89.8525) (end 174.3075 89.8525) (width 0.762) (layer B.Cu) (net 9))
 (segment (start 174.3075 89.8525) (end 175.26 88.9) (width 0.762) (layer B.Cu) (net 9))
 (segment (start 177.8 88.9) (end 179.07 90.17) (width 0.762) (layer B.Cu) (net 9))
 (segment (start 175.26 88.9) (end 177.8 88.9) (width 0.762) (layer B.Cu) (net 9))
 (segment (start 170.18 88.9) (end 170.815 88.9) (width 0.762) (layer B.Cu) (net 9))
 (segment (start 178.435 92.71) (end 179.07 92.075) (width 1.016) (layer B.Cu) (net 9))
 (segment (start 179.07 92.075) (end 179.07 90.17) (width 1.016) (layer B.Cu) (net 9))
 (segment (start 178.435 93.98) (end 178.435 92.71) (width 1.016) (layer B.Cu) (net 9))
 (segment (start 173.355 86.36) (end 173.355 87.63) (width 1.016) (layer B.Cu) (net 10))
 (segment (start 173.355 85.09) (end 173.355 86.36) (width 1.016) (layer B.Cu) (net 10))
 (segment (start 172.085 86.36) (end 173.355 86.36) (width 1.016) (layer B.Cu) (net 10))
 (segment (start 170.18 86.36) (end 172.085 86.36) (width 1.016) (layer B.Cu) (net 10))
 (segment (start 186.69 90.17) (end 189.23 90.17) (width 1.27) (layer B.Cu) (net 12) (status 20))
 (segment (start 162.56 86.36) (end 161.29 86.36) (width 0.762) (layer B.Cu) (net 6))
 (segment (start 161.29 86.36) (end 157.48 90.17) (width 0.762) (layer B.Cu) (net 6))
 (segment (start 157.48 90.17) (end 161.29 86.36) (width 0.508) (layer B.Cu) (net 6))
 (segment (start 170.18 91.44) (end 175.895 91.44) (width 0.762) (layer B.Cu) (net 8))
 (segment (start 197.612 88.392) (end 193.04 83.82) (width 1.27) (layer B.Cu) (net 11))
 (segment (start 193.04 83.82) (end 190.5 83.82) (width 1.27) (layer B.Cu) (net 11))
 (segment (start 198.882 89.662) (end 197.866 88.646) (width 1.27) (layer B.Cu) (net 11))
 (segment (start 197.866 88.646) (end 197.612 88.392) (width 1.27) (layer B.Cu) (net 11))
 (segment (start 201.295 93.98) (end 201.295 92.075) (width 1.27) (layer B.Cu) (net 11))
 (segment (start 198.12 88.9) (end 196.85 90.17) (width 1.27) (layer B.Cu) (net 11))
 (segment (start 201.295 92.075) (end 198.12 88.9) (width 1.27) (layer B.Cu) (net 11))
 (segment (start 201.295 93.98) (end 201.295 105.029) (width 1.27) (layer B.Cu) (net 11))
 (segment (start 201.295 105.029) (end 198.882 107.442) (width 1.27) (layer B.Cu) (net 11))
 (segment (start 180.848 120.396) (end 185.928 120.396) (width 1.27) (layer B.Cu) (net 11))
 (segment (start 198.882 107.442) (end 185.928 120.396) (width 1.27) (layer B.Cu) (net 11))
 (segment (start 179.54 124) (end 179.54 121.704) (width 1.27) (layer B.Cu) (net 11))
 (segment (start 179.54 121.704) (end 180.848 120.396) (width 1.27) (layer B.Cu) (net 11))
 (segment (start 177.165 83.82) (end 178.435 85.09) (width 1.27) (layer B.Cu) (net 13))
 (segment (start 178.435 85.09) (end 180.34 85.09) (width 1.27) (layer B.Cu) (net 13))
 (segment (start 175.895 83.82) (end 177.165 83.82) (width 1.27) (layer B.Cu) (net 13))
 (segment (start 157.48 92.71) (end 157.48 95.25) (width 1.27) (layer B.Cu) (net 14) (status 20)))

